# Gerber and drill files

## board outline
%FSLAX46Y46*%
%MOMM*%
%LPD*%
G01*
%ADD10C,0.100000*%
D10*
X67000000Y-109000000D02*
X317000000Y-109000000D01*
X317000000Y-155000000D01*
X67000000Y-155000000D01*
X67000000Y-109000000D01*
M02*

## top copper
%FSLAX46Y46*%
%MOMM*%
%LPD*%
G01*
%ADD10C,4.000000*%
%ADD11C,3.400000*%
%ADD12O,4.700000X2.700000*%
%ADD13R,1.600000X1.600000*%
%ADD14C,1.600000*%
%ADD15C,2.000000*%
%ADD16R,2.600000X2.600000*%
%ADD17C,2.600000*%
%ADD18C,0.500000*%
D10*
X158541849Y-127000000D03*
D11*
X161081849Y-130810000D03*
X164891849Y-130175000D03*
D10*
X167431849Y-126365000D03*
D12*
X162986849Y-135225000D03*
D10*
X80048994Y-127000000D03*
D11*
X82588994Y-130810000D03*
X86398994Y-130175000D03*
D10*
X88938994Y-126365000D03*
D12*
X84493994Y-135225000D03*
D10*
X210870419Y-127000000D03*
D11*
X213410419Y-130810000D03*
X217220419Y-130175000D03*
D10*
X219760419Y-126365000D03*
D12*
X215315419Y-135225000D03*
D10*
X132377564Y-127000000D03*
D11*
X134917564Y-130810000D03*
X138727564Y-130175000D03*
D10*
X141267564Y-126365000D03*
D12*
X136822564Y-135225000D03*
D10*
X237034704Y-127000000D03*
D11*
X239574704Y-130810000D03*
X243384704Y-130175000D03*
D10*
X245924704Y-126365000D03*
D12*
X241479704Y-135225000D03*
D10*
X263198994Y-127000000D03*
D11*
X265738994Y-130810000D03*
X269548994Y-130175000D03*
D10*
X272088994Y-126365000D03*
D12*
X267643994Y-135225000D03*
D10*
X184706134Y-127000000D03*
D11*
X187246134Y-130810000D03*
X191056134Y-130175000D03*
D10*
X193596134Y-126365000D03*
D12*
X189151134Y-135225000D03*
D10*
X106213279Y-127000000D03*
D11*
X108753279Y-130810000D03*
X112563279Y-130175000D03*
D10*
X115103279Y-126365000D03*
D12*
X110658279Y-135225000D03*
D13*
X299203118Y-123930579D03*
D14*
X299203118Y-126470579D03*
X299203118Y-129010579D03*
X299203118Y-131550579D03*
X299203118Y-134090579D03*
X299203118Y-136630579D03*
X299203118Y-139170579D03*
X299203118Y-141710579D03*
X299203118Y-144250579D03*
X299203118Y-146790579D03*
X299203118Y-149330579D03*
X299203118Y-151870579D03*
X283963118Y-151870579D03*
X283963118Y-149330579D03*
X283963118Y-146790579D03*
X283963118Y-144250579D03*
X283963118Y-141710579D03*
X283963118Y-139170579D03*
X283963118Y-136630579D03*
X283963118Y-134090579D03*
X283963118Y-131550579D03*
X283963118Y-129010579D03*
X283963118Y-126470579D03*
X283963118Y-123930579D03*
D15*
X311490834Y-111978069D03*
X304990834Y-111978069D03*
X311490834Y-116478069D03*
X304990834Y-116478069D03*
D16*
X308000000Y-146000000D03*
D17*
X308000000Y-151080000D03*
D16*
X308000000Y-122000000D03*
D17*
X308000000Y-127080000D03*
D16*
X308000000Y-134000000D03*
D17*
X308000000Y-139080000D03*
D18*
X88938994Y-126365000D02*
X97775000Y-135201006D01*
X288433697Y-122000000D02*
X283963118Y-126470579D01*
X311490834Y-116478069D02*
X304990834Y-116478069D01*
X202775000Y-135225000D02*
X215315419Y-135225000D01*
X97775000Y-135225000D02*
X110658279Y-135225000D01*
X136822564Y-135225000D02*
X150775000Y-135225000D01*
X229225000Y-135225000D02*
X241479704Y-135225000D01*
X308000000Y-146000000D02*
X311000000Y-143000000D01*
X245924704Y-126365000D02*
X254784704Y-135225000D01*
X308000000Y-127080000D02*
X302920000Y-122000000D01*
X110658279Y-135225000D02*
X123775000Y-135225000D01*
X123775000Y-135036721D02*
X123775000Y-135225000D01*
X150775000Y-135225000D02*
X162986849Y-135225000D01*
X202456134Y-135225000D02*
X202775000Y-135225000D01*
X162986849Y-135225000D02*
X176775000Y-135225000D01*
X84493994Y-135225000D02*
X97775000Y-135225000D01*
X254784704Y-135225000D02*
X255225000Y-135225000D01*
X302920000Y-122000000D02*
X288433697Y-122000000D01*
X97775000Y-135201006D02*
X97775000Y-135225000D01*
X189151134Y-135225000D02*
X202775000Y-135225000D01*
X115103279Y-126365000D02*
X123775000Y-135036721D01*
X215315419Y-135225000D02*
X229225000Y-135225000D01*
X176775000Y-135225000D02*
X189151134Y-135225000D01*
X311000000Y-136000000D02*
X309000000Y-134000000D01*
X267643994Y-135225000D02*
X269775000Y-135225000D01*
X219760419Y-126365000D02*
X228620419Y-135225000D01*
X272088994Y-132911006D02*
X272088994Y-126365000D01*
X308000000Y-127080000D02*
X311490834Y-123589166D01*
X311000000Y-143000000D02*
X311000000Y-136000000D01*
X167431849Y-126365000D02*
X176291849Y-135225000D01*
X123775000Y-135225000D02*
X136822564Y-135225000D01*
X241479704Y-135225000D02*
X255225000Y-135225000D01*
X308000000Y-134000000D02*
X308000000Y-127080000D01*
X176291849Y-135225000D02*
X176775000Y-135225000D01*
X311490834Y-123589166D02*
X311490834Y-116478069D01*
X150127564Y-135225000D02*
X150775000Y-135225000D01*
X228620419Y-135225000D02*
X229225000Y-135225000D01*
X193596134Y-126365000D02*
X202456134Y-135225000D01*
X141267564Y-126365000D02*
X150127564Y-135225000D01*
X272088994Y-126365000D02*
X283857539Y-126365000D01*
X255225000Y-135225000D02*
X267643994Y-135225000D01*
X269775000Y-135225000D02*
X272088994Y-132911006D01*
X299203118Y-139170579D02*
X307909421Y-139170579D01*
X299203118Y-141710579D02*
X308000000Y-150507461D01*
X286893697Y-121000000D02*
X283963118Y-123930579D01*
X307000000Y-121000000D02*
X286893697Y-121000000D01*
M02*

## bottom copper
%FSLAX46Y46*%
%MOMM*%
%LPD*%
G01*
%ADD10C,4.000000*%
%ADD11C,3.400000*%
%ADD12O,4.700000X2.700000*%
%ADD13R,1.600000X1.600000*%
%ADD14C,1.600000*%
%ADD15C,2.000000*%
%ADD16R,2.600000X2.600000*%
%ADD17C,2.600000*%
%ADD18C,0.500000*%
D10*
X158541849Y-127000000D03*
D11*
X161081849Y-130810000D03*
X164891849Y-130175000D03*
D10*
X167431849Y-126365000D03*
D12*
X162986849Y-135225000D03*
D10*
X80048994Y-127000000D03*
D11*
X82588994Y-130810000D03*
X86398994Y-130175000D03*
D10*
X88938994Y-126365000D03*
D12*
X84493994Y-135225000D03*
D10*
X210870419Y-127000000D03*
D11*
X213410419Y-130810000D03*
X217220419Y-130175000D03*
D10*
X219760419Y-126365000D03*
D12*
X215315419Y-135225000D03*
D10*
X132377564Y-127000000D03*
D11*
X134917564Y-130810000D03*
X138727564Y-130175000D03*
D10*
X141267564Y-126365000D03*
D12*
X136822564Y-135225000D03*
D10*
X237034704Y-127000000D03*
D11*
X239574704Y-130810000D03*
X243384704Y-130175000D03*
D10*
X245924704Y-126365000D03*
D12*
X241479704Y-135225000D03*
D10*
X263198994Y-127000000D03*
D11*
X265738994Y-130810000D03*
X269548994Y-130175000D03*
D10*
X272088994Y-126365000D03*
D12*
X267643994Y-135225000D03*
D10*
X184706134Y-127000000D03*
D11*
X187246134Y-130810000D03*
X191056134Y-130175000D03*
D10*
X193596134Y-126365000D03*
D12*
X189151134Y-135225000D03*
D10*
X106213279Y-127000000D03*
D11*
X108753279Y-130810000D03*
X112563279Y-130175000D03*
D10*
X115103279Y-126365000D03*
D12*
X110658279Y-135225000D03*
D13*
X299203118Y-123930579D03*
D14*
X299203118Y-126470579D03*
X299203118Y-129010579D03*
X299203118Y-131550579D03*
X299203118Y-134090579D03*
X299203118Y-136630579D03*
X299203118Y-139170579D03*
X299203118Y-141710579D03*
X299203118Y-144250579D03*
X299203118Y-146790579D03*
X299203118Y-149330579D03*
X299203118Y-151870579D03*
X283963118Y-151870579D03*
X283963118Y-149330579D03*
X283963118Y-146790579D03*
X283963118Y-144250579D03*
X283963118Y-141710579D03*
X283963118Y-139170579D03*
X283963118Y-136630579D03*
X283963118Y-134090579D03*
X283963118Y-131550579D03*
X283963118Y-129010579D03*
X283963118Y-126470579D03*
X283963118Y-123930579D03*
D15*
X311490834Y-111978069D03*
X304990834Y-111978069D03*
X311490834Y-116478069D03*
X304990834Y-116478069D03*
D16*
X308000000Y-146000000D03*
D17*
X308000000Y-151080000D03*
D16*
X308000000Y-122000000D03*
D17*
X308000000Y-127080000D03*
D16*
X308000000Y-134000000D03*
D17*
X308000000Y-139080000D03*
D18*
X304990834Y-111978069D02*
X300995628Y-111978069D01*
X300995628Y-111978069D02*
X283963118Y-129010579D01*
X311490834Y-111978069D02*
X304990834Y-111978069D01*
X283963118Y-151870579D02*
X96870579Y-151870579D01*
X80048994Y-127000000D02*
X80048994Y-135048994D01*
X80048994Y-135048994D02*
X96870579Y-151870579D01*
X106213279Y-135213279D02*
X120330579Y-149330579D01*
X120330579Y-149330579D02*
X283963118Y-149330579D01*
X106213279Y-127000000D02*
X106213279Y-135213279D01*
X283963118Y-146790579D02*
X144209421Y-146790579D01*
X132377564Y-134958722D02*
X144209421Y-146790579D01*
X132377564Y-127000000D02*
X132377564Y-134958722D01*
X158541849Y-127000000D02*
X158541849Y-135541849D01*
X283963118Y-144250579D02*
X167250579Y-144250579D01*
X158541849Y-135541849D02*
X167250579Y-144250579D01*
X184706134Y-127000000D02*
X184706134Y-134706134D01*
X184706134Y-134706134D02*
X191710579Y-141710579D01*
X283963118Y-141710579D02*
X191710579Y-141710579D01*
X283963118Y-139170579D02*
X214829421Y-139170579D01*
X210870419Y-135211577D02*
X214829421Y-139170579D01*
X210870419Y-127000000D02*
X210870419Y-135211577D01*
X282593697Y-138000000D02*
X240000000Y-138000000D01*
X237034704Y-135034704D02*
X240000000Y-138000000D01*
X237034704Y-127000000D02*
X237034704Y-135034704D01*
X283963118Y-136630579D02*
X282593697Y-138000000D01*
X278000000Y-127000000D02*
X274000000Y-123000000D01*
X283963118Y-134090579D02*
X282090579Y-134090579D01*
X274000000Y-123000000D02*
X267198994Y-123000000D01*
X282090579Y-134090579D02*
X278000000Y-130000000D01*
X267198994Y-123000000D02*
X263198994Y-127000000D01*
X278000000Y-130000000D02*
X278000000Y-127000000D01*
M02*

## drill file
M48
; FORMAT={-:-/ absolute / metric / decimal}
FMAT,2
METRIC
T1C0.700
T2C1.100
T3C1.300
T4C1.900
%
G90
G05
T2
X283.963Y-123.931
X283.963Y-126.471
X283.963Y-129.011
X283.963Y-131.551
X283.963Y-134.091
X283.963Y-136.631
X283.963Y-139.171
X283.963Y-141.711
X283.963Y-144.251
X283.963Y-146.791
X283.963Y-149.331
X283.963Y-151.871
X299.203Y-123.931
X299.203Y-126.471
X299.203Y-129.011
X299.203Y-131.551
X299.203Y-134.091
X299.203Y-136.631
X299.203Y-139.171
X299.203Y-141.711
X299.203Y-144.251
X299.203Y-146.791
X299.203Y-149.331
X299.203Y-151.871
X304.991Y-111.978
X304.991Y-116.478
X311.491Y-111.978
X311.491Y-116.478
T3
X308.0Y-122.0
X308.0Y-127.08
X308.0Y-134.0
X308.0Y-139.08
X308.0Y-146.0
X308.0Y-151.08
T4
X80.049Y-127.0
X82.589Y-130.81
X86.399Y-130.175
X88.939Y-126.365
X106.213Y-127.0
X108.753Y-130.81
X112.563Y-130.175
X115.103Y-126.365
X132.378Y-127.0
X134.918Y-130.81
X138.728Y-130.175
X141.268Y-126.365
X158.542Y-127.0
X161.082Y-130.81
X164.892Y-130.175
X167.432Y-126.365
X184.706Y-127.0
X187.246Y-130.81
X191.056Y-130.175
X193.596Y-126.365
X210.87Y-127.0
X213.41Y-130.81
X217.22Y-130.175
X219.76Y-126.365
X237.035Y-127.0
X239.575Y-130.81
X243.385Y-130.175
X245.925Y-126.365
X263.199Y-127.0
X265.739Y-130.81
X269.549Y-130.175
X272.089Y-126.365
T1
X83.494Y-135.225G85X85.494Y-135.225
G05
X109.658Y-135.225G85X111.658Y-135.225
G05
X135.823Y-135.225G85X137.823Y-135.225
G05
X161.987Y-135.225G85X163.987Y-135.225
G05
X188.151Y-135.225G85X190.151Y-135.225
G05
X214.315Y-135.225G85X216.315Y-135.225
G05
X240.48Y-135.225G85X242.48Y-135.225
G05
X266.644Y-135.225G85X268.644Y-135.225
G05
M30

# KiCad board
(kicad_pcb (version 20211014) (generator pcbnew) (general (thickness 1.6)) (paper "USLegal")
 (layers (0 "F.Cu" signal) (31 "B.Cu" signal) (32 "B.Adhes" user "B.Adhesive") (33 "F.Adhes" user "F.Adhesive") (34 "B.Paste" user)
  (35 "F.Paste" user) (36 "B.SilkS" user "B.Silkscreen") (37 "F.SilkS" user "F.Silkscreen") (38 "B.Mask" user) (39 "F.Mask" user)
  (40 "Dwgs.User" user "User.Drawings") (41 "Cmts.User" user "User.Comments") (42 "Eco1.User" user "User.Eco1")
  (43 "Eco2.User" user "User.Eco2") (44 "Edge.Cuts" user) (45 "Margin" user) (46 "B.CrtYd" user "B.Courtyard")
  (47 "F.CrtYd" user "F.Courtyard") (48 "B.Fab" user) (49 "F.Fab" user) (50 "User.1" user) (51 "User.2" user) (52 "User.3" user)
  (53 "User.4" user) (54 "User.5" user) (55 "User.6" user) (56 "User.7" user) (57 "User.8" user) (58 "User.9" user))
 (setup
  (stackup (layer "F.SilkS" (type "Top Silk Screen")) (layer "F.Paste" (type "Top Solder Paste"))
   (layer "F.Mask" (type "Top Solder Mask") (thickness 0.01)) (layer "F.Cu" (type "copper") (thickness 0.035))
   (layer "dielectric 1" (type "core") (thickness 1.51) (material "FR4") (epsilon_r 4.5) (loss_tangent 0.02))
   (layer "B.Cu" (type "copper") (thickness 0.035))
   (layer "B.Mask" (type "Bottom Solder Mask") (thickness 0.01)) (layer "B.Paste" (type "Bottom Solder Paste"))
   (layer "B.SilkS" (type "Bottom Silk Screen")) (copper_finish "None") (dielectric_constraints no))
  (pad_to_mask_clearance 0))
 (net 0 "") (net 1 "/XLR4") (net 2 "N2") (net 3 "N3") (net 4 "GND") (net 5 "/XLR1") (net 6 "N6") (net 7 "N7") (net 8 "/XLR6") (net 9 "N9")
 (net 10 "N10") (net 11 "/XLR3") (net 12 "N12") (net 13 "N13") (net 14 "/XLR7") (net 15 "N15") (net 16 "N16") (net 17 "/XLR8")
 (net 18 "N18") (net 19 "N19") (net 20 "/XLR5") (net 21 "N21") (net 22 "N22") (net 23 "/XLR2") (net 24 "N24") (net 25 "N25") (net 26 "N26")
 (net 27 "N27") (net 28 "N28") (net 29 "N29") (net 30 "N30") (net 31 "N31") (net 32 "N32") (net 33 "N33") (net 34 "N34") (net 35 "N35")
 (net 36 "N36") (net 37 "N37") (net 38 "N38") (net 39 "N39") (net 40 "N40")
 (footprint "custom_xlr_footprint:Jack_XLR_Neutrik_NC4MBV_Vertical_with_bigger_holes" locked (layer "F.Cu") (at 158.541849 127)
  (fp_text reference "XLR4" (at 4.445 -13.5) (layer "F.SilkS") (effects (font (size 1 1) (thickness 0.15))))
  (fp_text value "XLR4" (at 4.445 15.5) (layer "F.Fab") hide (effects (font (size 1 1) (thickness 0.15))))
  (pad "1" thru_hole circle locked (at 0 0) (size 4 4) (drill 1.9) (layers *.Cu *.Mask) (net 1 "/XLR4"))
  (pad "2" thru_hole circle locked (at 2.54 3.81) (size 3.4 3.4) (drill 1.9) (layers *.Cu *.Mask) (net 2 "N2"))
  (pad "3" thru_hole circle locked (at 6.35 3.175) (size 3.4 3.4) (drill 1.9) (layers *.Cu *.Mask) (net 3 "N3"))
  (pad "4" thru_hole circle locked (at 8.89 -0.635) (size 4 4) (drill 1.9) (layers *.Cu *.Mask) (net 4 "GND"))
  (pad "G" thru_hole oval locked (at 4.445 8.225) (size 4.7 2.7) (drill oval 2.7 0.7) (layers *.Cu *.Mask) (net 4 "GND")))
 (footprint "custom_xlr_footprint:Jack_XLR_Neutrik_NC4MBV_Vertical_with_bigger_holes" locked (layer "F.Cu") (at 80.048994 127)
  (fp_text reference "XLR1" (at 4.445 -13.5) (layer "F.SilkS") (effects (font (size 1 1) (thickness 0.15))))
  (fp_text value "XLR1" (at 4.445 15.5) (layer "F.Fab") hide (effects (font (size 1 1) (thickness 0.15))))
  (pad "1" thru_hole circle locked (at 0 0) (size 4 4) (drill 1.9) (layers *.Cu *.Mask) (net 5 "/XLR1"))
  (pad "2" thru_hole circle locked (at 2.54 3.81) (size 3.4 3.4) (drill 1.9) (layers *.Cu *.Mask) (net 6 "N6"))
  (pad "3" thru_hole circle locked (at 6.35 3.175) (size 3.4 3.4) (drill 1.9) (layers *.Cu *.Mask) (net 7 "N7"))
  (pad "4" thru_hole circle locked (at 8.89 -0.635) (size 4 4) (drill 1.9) (layers *.Cu *.Mask) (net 4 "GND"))
  (pad "G" thru_hole oval locked (at 4.445 8.225) (size 4.7 2.7) (drill oval 2.7 0.7) (layers *.Cu *.Mask) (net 4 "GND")))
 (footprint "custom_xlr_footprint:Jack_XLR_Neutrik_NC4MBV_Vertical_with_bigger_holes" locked (layer "F.Cu") (at 210.870419 127)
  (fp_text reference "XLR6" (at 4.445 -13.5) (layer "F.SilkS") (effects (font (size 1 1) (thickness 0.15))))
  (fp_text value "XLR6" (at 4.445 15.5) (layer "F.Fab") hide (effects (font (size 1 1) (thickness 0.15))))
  (pad "1" thru_hole circle locked (at 0 0) (size 4 4) (drill 1.9) (layers *.Cu *.Mask) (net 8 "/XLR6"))
  (pad "2" thru_hole circle locked (at 2.54 3.81) (size 3.4 3.4) (drill 1.9) (layers *.Cu *.Mask) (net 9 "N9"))
  (pad "3" thru_hole circle locked (at 6.35 3.175) (size 3.4 3.4) (drill 1.9) (layers *.Cu *.Mask) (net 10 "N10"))
  (pad "4" thru_hole circle locked (at 8.89 -0.635) (size 4 4) (drill 1.9) (layers *.Cu *.Mask) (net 4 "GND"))
  (pad "G" thru_hole oval locked (at 4.445 8.225) (size 4.7 2.7) (drill oval 2.7 0.7) (layers *.Cu *.Mask) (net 4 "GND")))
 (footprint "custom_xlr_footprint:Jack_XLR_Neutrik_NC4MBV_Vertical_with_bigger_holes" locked (layer "F.Cu") (at 132.377564 127)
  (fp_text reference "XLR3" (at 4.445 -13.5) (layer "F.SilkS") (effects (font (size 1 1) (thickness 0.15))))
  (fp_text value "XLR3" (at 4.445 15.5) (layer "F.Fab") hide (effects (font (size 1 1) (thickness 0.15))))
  (pad "1" thru_hole circle locked (at 0 0) (size 4 4) (drill 1.9) (layers *.Cu *.Mask) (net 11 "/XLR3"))
  (pad "2" thru_hole circle locked (at 2.54 3.81) (size 3.4 3.4) (drill 1.9) (layers *.Cu *.Mask) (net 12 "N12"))
  (pad "3" thru_hole circle locked (at 6.35 3.175) (size 3.4 3.4) (drill 1.9) (layers *.Cu *.Mask) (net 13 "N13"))
  (pad "4" thru_hole circle locked (at 8.89 -0.635) (size 4 4) (drill 1.9) (layers *.Cu *.Mask) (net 4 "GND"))
  (pad "G" thru_hole oval locked (at 4.445 8.225) (size 4.7 2.7) (drill oval 2.7 0.7) (layers *.Cu *.Mask) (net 4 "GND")))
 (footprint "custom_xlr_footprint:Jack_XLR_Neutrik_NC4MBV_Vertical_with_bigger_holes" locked (layer "F.Cu") (at 237.034704 127)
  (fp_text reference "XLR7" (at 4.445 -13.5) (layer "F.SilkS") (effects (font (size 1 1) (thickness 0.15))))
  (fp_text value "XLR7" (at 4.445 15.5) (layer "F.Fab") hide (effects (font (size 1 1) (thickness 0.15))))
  (pad "1" thru_hole circle locked (at 0 0) (size 4 4) (drill 1.9) (layers *.Cu *.Mask) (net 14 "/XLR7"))
  (pad "2" thru_hole circle locked (at 2.54 3.81) (size 3.4 3.4) (drill 1.9) (layers *.Cu *.Mask) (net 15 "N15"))
  (pad "3" thru_hole circle locked (at 6.35 3.175) (size 3.4 3.4) (drill 1.9) (layers *.Cu *.Mask) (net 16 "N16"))
  (pad "4" thru_hole circle locked (at 8.89 -0.635) (size 4 4) (drill 1.9) (layers *.Cu *.Mask) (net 4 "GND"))
  (pad "G" thru_hole oval locked (at 4.445 8.225) (size 4.7 2.7) (drill oval 2.7 0.7) (layers *.Cu *.Mask) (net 4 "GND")))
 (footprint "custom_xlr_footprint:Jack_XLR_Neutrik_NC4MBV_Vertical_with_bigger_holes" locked (layer "F.Cu") (at 263.198994 127)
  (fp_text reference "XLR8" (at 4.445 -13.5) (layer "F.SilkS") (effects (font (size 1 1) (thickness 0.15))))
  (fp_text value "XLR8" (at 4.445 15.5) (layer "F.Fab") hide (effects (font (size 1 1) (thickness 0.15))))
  (pad "1" thru_hole circle locked (at 0 0) (size 4 4) (drill 1.9) (layers *.Cu *.Mask) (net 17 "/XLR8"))
  (pad "2" thru_hole circle locked (at 2.54 3.81) (size 3.4 3.4) (drill 1.9) (layers *.Cu *.Mask) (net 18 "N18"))
  (pad "3" thru_hole circle locked (at 6.35 3.175) (size 3.4 3.4) (drill 1.9) (layers *.Cu *.Mask) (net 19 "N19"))
  (pad "4" thru_hole circle locked (at 8.89 -0.635) (size 4 4) (drill 1.9) (layers *.Cu *.Mask) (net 4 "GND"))
  (pad "G" thru_hole oval locked (at 4.445 8.225) (size 4.7 2.7) (drill oval 2.7 0.7) (layers *.Cu *.Mask) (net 4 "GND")))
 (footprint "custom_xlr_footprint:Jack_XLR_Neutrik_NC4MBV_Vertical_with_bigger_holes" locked (layer "F.Cu") (at 184.706134 127)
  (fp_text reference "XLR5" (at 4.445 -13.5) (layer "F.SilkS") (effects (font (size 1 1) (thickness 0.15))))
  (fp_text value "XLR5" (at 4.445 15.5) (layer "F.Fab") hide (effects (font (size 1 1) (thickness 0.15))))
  (pad "1" thru_hole circle locked (at 0 0) (size 4 4) (drill 1.9) (layers *.Cu *.Mask) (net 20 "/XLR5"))
  (pad "2" thru_hole circle locked (at 2.54 3.81) (size 3.4 3.4) (drill 1.9) (layers *.Cu *.Mask) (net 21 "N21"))
  (pad "3" thru_hole circle locked (at 6.35 3.175) (size 3.4 3.4) (drill 1.9) (layers *.Cu *.Mask) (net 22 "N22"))
  (pad "4" thru_hole circle locked (at 8.89 -0.635) (size 4 4) (drill 1.9) (layers *.Cu *.Mask) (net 4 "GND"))
  (pad "G" thru_hole oval locked (at 4.445 8.225) (size 4.7 2.7) (drill oval 2.7 0.7) (layers *.Cu *.Mask) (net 4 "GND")))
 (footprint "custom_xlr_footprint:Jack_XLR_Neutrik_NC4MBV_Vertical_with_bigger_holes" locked (layer "F.Cu") (at 106.213279 127)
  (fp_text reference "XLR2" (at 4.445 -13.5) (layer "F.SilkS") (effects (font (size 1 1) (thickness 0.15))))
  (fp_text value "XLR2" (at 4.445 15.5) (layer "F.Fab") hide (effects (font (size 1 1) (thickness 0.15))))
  (pad "1" thru_hole circle locked (at 0 0) (size 4 4) (drill 1.9) (layers *.Cu *.Mask) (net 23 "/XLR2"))
  (pad "2" thru_hole circle locked (at 2.54 3.81) (size 3.4 3.4) (drill 1.9) (layers *.Cu *.Mask) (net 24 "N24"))
  (pad "3" thru_hole circle locked (at 6.35 3.175) (size 3.4 3.4) (drill 1.9) (layers *.Cu *.Mask) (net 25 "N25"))
  (pad "4" thru_hole circle locked (at 8.89 -0.635) (size 4 4) (drill 1.9) (layers *.Cu *.Mask) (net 4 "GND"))
  (pad "G" thru_hole oval locked (at 4.445 8.225) (size 4.7 2.7) (drill oval 2.7 0.7) (layers *.Cu *.Mask) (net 4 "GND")))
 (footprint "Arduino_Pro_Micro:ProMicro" (layer "B.Cu") (at 291.583118 137.900579 -90)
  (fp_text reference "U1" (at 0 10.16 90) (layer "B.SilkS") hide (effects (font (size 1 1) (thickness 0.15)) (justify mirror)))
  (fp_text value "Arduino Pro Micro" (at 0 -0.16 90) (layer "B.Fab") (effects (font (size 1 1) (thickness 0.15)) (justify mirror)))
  (pad "1" thru_hole rect locked (at -13.97 -7.62 270) (size 1.6 1.6) (drill 1.1) (layers *.Cu *.Mask "B.SilkS") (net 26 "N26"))
  (pad "2" thru_hole circle locked (at -11.43 -7.62 270) (size 1.6 1.6) (drill 1.1) (layers *.Cu *.Mask "B.SilkS") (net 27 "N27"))
  (pad "3" thru_hole circle locked (at -8.89 -7.62 270) (size 1.6 1.6) (drill 1.1) (layers *.Cu *.Mask "B.SilkS") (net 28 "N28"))
  (pad "4" thru_hole circle locked (at -6.35 -7.62 270) (size 1.6 1.6) (drill 1.1) (layers *.Cu *.Mask "B.SilkS") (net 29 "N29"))
  (pad "5" thru_hole circle locked (at -3.81 -7.62 270) (size 1.6 1.6) (drill 1.1) (layers *.Cu *.Mask "B.SilkS") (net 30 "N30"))
  (pad "6" thru_hole circle locked (at -1.27 -7.62 270) (size 1.6 1.6) (drill 1.1) (layers *.Cu *.Mask "B.SilkS") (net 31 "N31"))
  (pad "7" thru_hole circle locked (at 1.27 -7.62 270) (size 1.6 1.6) (drill 1.1) (layers *.Cu *.Mask "B.SilkS") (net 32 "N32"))
  (pad "8" thru_hole circle locked (at 3.81 -7.62 270) (size 1.6 1.6) (drill 1.1) (layers *.Cu *.Mask "B.SilkS") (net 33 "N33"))
  (pad "9" thru_hole circle locked (at 6.35 -7.62 270) (size 1.6 1.6) (drill 1.1) (layers *.Cu *.Mask "B.SilkS") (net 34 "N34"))
  (pad "10" thru_hole circle locked (at 8.89 -7.62 270) (size 1.6 1.6) (drill 1.1) (layers *.Cu *.Mask "B.SilkS") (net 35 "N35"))
  (pad "11" thru_hole circle locked (at 11.43 -7.62 270) (size 1.6 1.6) (drill 1.1) (layers *.Cu *.Mask "B.SilkS") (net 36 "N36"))
  (pad "12" thru_hole circle locked (at 13.97 -7.62 270) (size 1.6 1.6) (drill 1.1) (layers *.Cu *.Mask "B.SilkS") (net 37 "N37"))
  (pad "13" thru_hole circle locked (at 13.97 7.62 270) (size 1.6 1.6) (drill 1.1) (layers *.Cu *.Mask "B.SilkS") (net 5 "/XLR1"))
  (pad "14" thru_hole circle locked (at 11.43 7.62 270) (size 1.6 1.6) (drill 1.1) (layers *.Cu *.Mask "B.SilkS") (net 23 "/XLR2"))
  (pad "15" thru_hole circle locked (at 8.89 7.62 270) (size 1.6 1.6) (drill 1.1) (layers *.Cu *.Mask "B.SilkS") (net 11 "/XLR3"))
  (pad "16" thru_hole circle locked (at 6.35 7.62 270) (size 1.6 1.6) (drill 1.1) (layers *.Cu *.Mask "B.SilkS") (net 1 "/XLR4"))
  (pad "17" thru_hole circle locked (at 3.81 7.62 270) (size 1.6 1.6) (drill 1.1) (layers *.Cu *.Mask "B.SilkS") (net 20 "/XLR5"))
  (pad "18" thru_hole circle locked (at 1.27 7.62 270) (size 1.6 1.6) (drill 1.1) (layers *.Cu *.Mask "B.SilkS") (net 8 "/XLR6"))
  (pad "19" thru_hole circle locked (at -1.27 7.62 270) (size 1.6 1.6) (drill 1.1) (layers *.Cu *.Mask "B.SilkS") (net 14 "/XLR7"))
  (pad "20" thru_hole circle locked (at -3.81 7.62 270) (size 1.6 1.6) (drill 1.1) (layers *.Cu *.Mask "B.SilkS") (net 17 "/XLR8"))
  (pad "21" thru_hole circle locked (at -6.35 7.62 270) (size 1.6 1.6) (drill 1.1) (layers *.Cu *.Mask "B.SilkS") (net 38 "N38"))
  (pad "22" thru_hole circle locked (at -8.89 7.62 270) (size 1.6 1.6) (drill 1.1) (layers *.Cu *.Mask "B.SilkS") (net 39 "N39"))
  (pad "23" thru_hole circle locked (at -11.43 7.62 270) (size 1.6 1.6) (drill 1.1) (layers *.Cu *.Mask "B.SilkS") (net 4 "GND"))
  (pad "24" thru_hole circle locked (at -13.97 7.62 270) (size 1.6 1.6) (drill 1.1) (layers *.Cu *.Mask "B.SilkS") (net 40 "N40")))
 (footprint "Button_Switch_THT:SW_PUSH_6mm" (layer "B.Cu") (at 311.490834 111.978069 180)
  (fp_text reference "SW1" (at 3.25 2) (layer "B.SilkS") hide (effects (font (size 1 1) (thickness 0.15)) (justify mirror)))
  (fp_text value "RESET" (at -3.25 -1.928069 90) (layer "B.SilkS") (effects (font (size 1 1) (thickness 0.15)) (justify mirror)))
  (pad "1" thru_hole circle (at 0 0 90) (size 2 2) (drill 1.1) (layers *.Cu *.Mask) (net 39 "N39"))
  (pad "1" thru_hole circle (at 6.5 0 90) (size 2 2) (drill 1.1) (layers *.Cu *.Mask) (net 39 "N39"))
  (pad "2" thru_hole circle (at 0 -4.5 90) (size 2 2) (drill 1.1) (layers *.Cu *.Mask) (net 4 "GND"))
  (pad "2" thru_hole circle (at 6.5 -4.5 90) (size 2 2) (drill 1.1) (layers *.Cu *.Mask) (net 4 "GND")))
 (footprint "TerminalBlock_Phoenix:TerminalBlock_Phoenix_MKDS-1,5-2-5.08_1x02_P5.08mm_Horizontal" (layer "B.Cu") (at 308 146 -90)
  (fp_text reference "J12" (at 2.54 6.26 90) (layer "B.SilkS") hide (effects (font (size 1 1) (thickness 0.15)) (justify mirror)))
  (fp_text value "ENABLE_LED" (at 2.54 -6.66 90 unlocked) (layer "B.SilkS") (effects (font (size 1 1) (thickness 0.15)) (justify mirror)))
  (pad "1" thru_hole rect (at 0 0 270) (size 2.6 2.6) (drill 1.3) (layers *.Cu *.Mask) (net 4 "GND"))
  (pad "2" thru_hole circle (at 5.08 0 270) (size 2.6 2.6) (drill 1.3) (layers *.Cu *.Mask) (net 33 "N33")))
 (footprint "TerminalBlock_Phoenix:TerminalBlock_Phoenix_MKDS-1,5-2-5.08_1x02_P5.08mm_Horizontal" (layer "B.Cu") (at 308 122 -90)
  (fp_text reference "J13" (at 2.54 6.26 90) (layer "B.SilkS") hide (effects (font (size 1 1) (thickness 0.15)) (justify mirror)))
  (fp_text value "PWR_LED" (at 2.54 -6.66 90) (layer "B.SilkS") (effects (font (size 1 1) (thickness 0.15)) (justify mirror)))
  (pad "1" thru_hole rect (at 0 0 270) (size 2.6 2.6) (drill 1.3) (layers *.Cu *.Mask) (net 40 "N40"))
  (pad "2" thru_hole circle (at 5.08 0 270) (size 2.6 2.6) (drill 1.3) (layers *.Cu *.Mask) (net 4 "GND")))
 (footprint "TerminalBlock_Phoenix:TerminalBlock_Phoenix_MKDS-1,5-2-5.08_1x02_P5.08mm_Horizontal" (layer "B.Cu") (at 308 134 -90)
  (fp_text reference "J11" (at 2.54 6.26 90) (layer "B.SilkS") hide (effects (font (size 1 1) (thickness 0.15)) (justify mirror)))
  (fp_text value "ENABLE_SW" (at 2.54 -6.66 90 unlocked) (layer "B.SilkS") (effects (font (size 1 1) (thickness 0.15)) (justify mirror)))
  (pad "1" thru_hole rect (at 0 0 270) (size 2.6 2.6) (drill 1.3) (layers *.Cu *.Mask) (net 4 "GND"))
  (pad "2" thru_hole circle (at 5.08 0 270) (size 2.6 2.6) (drill 1.3) (layers *.Cu *.Mask) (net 32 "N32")))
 (gr_rect (start 67 109) (end 317 155) (layer "Edge.Cuts") (width 0.1) (fill none))
 (segment (start 88.938994 126.365) (end 97.775 135.201006) (width 0.5) (layer "F.Cu") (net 4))
 (segment (start 288.433697 122) (end 283.963118 126.470579) (width 0.5) (layer "F.Cu") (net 4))
 (segment (start 311.490834 116.478069) (end 304.990834 116.478069) (width 0.5) (layer "F.Cu") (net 4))
 (segment (start 202.775 135.225) (end 215.315419 135.225) (width 0.5) (layer "F.Cu") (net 4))
 (segment (start 97.775 135.225) (end 110.658279 135.225) (width 0.5) (layer "F.Cu") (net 4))
 (segment (start 136.822564 135.225) (end 150.775 135.225) (width 0.5) (layer "F.Cu") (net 4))
 (segment (start 229.225 135.225) (end 241.479704 135.225) (width 0.5) (layer "F.Cu") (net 4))
 (segment (start 308 146) (end 311 143) (width 0.5) (layer "F.Cu") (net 4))
 (segment (start 245.924704 126.365) (end 254.784704 135.225) (width 0.5) (layer "F.Cu") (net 4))
 (segment (start 308 127.08) (end 302.92 122) (width 0.5) (layer "F.Cu") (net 4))
 (segment (start 110.658279 135.225) (end 123.775 135.225) (width 0.5) (layer "F.Cu") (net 4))
 (segment (start 123.775 135.036721) (end 123.775 135.225) (width 0.5) (layer "F.Cu") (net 4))
 (segment (start 150.775 135.225) (end 162.986849 135.225) (width 0.5) (layer "F.Cu") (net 4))
 (segment (start 202.456134 135.225) (end 202.775 135.225) (width 0.5) (layer "F.Cu") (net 4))
 (segment (start 162.986849 135.225) (end 176.775 135.225) (width 0.5) (layer "F.Cu") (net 4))
 (segment (start 84.493994 135.225) (end 97.775 135.225) (width 0.5) (layer "F.Cu") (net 4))
 (segment (start 254.784704 135.225) (end 255.225 135.225) (width 0.5) (layer "F.Cu") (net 4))
 (segment (start 302.92 122) (end 288.433697 122) (width 0.5) (layer "F.Cu") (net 4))
 (segment (start 97.775 135.201006) (end 97.775 135.225) (width 0.5) (layer "F.Cu") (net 4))
 (segment (start 189.151134 135.225) (end 202.775 135.225) (width 0.5) (layer "F.Cu") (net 4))
 (segment (start 115.103279 126.365) (end 123.775 135.036721) (width 0.5) (layer "F.Cu") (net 4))
 (segment (start 215.315419 135.225) (end 229.225 135.225) (width 0.5) (layer "F.Cu") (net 4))
 (segment (start 176.775 135.225) (end 189.151134 135.225) (width 0.5) (layer "F.Cu") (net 4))
 (segment (start 311 136) (end 309 134) (width 0.5) (layer "F.Cu") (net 4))
 (segment (start 267.643994 135.225) (end 269.775 135.225) (width 0.5) (layer "F.Cu") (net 4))
 (segment (start 219.760419 126.365) (end 228.620419 135.225) (width 0.5) (layer "F.Cu") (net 4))
 (segment (start 272.088994 132.911006) (end 272.088994 126.365) (width 0.5) (layer "F.Cu") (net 4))
 (segment (start 308 127.08) (end 311.490834 123.589166) (width 0.5) (layer "F.Cu") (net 4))
 (segment (start 311 143) (end 311 136) (width 0.5) (layer "F.Cu") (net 4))
 (segment (start 167.431849 126.365) (end 176.291849 135.225) (width 0.5) (layer "F.Cu") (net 4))
 (segment (start 123.775 135.225) (end 136.822564 135.225) (width 0.5) (layer "F.Cu") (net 4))
 (segment (start 241.479704 135.225) (end 255.225 135.225) (width 0.5) (layer "F.Cu") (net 4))
 (segment (start 308 134) (end 308 127.08) (width 0.5) (layer "F.Cu") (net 4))
 (segment (start 176.291849 135.225) (end 176.775 135.225) (width 0.5) (layer "F.Cu") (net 4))
 (segment (start 311.490834 123.589166) (end 311.490834 116.478069) (width 0.5) (layer "F.Cu") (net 4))
 (segment (start 150.127564 135.225) (end 150.775 135.225) (width 0.5) (layer "F.Cu") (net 4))
 (segment (start 228.620419 135.225) (end 229.225 135.225) (width 0.5) (layer "F.Cu") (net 4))
 (segment (start 193.596134 126.365) (end 202.456134 135.225) (width 0.5) (layer "F.Cu") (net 4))
 (segment (start 141.267564 126.365) (end 150.127564 135.225) (width 0.5) (layer "F.Cu") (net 4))
 (segment (start 272.088994 126.365) (end 283.857539 126.365) (width 0.5) (layer "F.Cu") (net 4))
 (segment (start 255.225 135.225) (end 267.643994 135.225) (width 0.5) (layer "F.Cu") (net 4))
 (segment (start 269.775 135.225) (end 272.088994 132.911006) (width 0.5) (layer "F.Cu") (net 4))
 (segment (start 299.203118 139.170579) (end 307.909421 139.170579) (width 0.5) (layer "F.Cu") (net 32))
 (segment (start 299.203118 141.710579) (end 308 150.507461) (width 0.5) (layer "F.Cu") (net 33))
 (segment (start 286.893697 121) (end 283.963118 123.930579) (width 0.5) (layer "F.Cu") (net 40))
 (segment (start 307 121) (end 286.893697 121) (width 0.5) (layer "F.Cu") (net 40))
 (segment (start 304.990834 111.978069) (end 300.995628 111.978069) (width 0.5) (layer "B.Cu") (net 39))
 (segment (start 300.995628 111.978069) (end 283.963118 129.010579) (width 0.5) (layer "B.Cu") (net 39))
 (segment (start 311.490834 111.978069) (end 304.990834 111.978069) (width 0.5) (layer "B.Cu") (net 39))
 (segment (start 283.963118 151.870579) (end 96.870579 151.870579) (width 0.5) (layer "B.Cu") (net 5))
 (segment (start 80.048994 127) (end 80.048994 135.048994) (width 0.5) (layer "B.Cu") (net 5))
 (segment (start 80.048994 135.048994) (end 96.870579 151.870579) (width 0.5) (layer "B.Cu") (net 5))
 (segment (start 106.213279 135.213279) (end 120.330579 149.330579) (width 0.5) (layer "B.Cu") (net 23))
 (segment (start 120.330579 149.330579) (end 283.963118 149.330579) (width 0.5) (layer "B.Cu") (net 23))
 (segment (start 106.213279 127) (end 106.213279 135.213279) (width 0.5) (layer "B.Cu") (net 23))
 (segment (start 283.963118 146.790579) (end 144.209421 146.790579) (width 0.5) (layer "B.Cu") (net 11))
 (segment (start 132.377564 134.958722) (end 144.209421 146.790579) (width 0.5) (layer "B.Cu") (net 11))
 (segment (start 132.377564 127) (end 132.377564 134.958722) (width 0.5) (layer "B.Cu") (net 11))
 (segment (start 158.541849 127) (end 158.541849 135.541849) (width 0.5) (layer "B.Cu") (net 1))
 (segment (start 283.963118 144.250579) (end 167.250579 144.250579) (width 0.5) (layer "B.Cu") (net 1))
 (segment (start 158.541849 135.541849) (end 167.250579 144.250579) (width 0.5) (layer "B.Cu") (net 1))
 (segment (start 184.706134 127) (end 184.706134 134.706134) (width 0.5) (layer "B.Cu") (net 20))
 (segment (start 184.706134 134.706134) (end 191.710579 141.710579) (width 0.5) (layer "B.Cu") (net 20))
 (segment (start 283.963118 141.710579) (end 191.710579 141.710579) (width 0.5) (layer "B.Cu") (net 20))
 (segment (start 283.963118 139.170579) (end 214.829421 139.170579) (width 0.5) (layer "B.Cu") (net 8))
 (segment (start 210.870419 135.211577) (end 214.829421 139.170579) (width 0.5) (layer "B.Cu") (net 8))
 (segment (start 210.870419 127) (end 210.870419 135.211577) (width 0.5) (layer "B.Cu") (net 8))
 (segment (start 282.593697 138) (end 240 138) (width 0.5) (layer "B.Cu") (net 14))
 (segment (start 237.034704 135.034704) (end 240 138) (width 0.5) (layer "B.Cu") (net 14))
 (segment (start 237.034704 127) (end 237.034704 135.034704) (width 0.5) (layer "B.Cu") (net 14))
 (segment (start 283.963118 136.630579) (end 282.593697 138) (width 0.5) (layer "B.Cu") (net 14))
 (segment (start 278 127) (end 274 123) (width 0.5) (layer "B.Cu") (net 17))
 (segment (start 283.963118 134.090579) (end 282.090579 134.090579) (width 0.5) (layer "B.Cu") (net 17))
 (segment (start 274 123) (end 267.198994 123) (width 0.5) (layer "B.Cu") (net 17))
 (segment (start 282.090579 134.090579) (end 278 130) (width 0.5) (layer "B.Cu") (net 17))
 (segment (start 267.198994 123) (end 263.198994 127) (width 0.5) (layer "B.Cu") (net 17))
 (segment (start 278 130) (end 278 127) (width 0.5) (layer "B.Cu") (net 17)))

